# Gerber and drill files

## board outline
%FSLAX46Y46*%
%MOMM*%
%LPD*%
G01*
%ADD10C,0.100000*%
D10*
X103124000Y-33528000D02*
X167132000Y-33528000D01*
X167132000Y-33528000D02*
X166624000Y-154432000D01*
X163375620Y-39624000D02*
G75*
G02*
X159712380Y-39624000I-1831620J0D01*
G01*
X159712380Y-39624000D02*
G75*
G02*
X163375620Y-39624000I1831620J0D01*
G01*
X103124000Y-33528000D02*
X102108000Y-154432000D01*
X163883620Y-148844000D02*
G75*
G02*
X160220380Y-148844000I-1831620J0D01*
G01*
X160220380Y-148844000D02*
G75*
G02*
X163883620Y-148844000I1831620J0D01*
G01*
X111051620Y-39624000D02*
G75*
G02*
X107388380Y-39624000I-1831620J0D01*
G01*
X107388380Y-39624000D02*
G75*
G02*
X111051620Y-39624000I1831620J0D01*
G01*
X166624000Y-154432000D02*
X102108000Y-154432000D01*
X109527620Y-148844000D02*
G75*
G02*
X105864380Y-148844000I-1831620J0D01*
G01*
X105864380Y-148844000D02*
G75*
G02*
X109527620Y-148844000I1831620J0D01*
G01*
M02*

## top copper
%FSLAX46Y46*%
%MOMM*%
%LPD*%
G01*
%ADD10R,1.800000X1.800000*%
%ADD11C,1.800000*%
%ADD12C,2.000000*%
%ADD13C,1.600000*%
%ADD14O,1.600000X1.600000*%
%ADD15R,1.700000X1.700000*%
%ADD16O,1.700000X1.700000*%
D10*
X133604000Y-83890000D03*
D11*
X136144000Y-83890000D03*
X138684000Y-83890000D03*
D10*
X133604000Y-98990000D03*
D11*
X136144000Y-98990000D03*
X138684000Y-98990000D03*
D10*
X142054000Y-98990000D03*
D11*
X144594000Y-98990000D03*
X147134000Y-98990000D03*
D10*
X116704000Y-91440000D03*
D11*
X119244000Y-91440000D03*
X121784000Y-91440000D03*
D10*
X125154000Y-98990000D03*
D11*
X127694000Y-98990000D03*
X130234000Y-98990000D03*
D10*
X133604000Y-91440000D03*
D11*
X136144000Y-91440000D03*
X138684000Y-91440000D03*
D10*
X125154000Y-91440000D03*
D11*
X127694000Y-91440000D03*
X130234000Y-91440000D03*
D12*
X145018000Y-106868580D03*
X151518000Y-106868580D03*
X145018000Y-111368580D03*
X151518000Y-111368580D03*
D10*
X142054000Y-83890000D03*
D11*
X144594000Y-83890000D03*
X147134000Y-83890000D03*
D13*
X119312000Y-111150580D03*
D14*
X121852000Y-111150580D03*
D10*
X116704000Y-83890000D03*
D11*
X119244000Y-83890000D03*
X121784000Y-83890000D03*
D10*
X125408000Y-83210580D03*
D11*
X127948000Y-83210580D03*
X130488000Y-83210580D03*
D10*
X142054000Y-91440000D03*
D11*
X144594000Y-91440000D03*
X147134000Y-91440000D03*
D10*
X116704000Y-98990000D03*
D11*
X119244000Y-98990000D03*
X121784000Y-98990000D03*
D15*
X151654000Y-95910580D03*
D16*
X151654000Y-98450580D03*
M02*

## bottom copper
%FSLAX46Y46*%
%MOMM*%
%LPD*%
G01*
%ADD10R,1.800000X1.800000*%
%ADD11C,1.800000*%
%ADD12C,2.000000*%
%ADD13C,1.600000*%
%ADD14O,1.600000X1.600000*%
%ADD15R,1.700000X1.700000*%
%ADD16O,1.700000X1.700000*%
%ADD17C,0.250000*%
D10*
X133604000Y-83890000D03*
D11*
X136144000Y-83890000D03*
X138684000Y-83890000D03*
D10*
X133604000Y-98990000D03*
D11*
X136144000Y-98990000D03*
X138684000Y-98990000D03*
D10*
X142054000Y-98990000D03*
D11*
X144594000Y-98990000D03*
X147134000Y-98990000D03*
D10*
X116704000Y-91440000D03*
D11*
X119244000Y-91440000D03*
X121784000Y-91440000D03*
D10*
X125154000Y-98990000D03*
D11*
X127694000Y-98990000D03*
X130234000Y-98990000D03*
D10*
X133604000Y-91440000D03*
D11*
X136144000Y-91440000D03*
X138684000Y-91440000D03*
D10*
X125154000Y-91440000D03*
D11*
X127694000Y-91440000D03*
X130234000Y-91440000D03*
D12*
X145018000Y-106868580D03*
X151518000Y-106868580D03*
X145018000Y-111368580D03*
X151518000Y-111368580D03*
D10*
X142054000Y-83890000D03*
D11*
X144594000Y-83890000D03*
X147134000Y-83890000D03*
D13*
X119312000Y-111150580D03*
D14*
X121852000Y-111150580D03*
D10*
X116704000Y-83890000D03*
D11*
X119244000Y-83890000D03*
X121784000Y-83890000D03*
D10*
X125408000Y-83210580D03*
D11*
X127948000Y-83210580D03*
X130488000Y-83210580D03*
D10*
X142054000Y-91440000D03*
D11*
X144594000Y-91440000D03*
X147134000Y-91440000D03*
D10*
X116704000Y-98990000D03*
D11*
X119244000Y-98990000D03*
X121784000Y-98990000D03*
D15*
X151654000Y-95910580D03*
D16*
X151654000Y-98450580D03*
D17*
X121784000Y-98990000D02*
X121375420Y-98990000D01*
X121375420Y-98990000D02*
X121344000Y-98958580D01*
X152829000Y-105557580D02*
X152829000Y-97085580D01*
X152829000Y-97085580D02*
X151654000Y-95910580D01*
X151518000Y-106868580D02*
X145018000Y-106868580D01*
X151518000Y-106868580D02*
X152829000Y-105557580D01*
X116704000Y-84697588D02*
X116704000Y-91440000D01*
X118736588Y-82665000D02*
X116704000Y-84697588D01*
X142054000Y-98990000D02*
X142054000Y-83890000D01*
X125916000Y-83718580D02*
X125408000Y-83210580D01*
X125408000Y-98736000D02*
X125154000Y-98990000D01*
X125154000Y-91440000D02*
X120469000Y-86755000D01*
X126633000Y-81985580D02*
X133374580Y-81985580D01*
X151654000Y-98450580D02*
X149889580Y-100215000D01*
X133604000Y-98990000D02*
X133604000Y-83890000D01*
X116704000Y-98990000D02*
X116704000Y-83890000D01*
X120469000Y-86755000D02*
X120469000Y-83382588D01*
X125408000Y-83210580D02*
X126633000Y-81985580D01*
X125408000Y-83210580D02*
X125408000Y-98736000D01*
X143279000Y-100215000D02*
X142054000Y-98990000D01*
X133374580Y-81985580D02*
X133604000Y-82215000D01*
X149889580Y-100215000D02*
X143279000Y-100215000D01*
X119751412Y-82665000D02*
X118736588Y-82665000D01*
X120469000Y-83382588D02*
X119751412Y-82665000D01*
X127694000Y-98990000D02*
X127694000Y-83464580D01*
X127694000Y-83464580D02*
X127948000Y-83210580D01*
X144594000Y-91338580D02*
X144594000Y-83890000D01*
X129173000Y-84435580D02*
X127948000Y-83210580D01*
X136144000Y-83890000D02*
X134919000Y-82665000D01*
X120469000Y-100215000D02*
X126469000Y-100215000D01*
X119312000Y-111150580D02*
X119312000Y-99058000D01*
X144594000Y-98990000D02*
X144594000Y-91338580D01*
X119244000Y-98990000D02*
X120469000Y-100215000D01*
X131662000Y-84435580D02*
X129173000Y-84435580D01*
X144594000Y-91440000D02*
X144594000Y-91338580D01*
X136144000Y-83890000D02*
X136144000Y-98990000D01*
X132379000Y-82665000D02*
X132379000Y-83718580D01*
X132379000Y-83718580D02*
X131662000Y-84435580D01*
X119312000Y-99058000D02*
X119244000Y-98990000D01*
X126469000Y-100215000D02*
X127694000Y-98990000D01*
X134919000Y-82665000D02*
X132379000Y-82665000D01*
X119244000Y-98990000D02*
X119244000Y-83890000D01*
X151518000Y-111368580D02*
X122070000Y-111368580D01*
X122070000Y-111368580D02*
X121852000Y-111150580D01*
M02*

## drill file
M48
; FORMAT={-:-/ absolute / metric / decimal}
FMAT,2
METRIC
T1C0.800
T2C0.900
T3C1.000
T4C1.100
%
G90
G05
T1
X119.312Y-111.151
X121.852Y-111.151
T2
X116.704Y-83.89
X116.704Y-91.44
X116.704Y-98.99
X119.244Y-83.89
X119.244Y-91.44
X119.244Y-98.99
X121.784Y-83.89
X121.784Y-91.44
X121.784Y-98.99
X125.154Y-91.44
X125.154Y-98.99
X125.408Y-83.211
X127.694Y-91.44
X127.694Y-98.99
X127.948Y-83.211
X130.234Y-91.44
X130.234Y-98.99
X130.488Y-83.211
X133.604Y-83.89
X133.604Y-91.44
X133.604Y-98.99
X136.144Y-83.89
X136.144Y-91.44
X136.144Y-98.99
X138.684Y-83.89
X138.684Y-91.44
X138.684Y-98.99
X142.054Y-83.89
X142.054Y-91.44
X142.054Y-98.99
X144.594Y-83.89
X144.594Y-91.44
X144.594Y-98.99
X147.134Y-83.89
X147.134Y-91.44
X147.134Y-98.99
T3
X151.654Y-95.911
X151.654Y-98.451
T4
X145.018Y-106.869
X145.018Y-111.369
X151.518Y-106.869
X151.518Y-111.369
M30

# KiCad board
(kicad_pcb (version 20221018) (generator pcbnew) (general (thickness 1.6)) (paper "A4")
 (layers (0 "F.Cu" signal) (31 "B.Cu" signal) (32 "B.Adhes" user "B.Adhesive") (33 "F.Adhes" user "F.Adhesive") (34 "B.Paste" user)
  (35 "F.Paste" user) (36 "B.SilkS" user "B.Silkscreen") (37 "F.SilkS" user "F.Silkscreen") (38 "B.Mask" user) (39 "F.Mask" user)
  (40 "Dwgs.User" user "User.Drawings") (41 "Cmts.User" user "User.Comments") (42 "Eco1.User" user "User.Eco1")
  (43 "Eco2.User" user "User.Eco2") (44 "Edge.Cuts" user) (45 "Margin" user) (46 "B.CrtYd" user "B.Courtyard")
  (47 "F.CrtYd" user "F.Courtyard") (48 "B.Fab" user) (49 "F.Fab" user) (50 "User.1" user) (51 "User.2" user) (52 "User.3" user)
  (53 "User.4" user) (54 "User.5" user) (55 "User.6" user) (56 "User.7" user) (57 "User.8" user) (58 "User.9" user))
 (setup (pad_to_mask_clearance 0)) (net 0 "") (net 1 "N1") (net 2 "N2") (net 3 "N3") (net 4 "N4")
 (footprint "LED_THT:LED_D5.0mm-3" (layer "F.Cu") (at 133.604 83.89)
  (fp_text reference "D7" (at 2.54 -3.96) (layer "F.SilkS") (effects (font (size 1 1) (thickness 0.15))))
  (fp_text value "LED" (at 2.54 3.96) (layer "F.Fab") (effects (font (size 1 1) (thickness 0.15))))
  (pad "1" thru_hole rect (at 0 0) (size 1.8 1.8) (drill 0.9) (layers "*.Cu" "*.Mask") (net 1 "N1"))
  (pad "2" thru_hole circle (at 2.54 0) (size 1.8 1.8) (drill 0.9) (layers "*.Cu" "*.Mask") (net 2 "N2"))
  (pad "3" thru_hole circle (at 5.08 0) (size 1.8 1.8) (drill 0.9) (layers "*.Cu" "*.Mask")))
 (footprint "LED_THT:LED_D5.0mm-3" (layer "F.Cu") (at 133.604 98.99)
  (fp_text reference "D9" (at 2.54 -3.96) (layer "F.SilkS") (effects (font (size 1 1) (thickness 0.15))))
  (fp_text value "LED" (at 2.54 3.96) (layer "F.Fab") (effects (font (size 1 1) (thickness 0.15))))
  (pad "1" thru_hole rect (at 0 0) (size 1.8 1.8) (drill 0.9) (layers "*.Cu" "*.Mask") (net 1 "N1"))
  (pad "2" thru_hole circle (at 2.54 0) (size 1.8 1.8) (drill 0.9) (layers "*.Cu" "*.Mask") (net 2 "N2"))
  (pad "3" thru_hole circle (at 5.08 0) (size 1.8 1.8) (drill 0.9) (layers "*.Cu" "*.Mask")))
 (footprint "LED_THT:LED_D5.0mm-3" (layer "F.Cu") (at 142.054 98.99)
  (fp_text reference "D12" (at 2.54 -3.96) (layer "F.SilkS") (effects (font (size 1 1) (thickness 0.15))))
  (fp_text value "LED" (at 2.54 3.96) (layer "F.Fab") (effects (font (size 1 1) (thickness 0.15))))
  (pad "1" thru_hole rect (at 0 0) (size 1.8 1.8) (drill 0.9) (layers "*.Cu" "*.Mask") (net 1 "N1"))
  (pad "2" thru_hole circle (at 2.54 0) (size 1.8 1.8) (drill 0.9) (layers "*.Cu" "*.Mask") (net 2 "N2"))
  (pad "3" thru_hole circle (at 5.08 0) (size 1.8 1.8) (drill 0.9) (layers "*.Cu" "*.Mask")))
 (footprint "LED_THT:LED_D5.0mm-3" (layer "F.Cu") (at 116.704 91.44)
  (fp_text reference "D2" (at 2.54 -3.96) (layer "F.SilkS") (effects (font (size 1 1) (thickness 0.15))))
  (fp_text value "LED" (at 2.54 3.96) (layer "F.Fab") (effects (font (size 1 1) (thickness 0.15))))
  (pad "1" thru_hole rect (at 0 0) (size 1.8 1.8) (drill 0.9) (layers "*.Cu" "*.Mask") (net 1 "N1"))
  (pad "2" thru_hole circle (at 2.54 0) (size 1.8 1.8) (drill 0.9) (layers "*.Cu" "*.Mask") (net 2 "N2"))
  (pad "3" thru_hole circle (at 5.08 0) (size 1.8 1.8) (drill 0.9) (layers "*.Cu" "*.Mask")))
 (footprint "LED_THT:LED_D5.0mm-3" (layer "F.Cu") (at 125.154 98.99)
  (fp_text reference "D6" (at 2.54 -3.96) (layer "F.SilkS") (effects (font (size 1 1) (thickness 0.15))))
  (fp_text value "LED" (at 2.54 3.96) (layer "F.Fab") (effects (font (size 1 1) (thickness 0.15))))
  (pad "1" thru_hole rect (at 0 0) (size 1.8 1.8) (drill 0.9) (layers "*.Cu" "*.Mask") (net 1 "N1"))
  (pad "2" thru_hole circle (at 2.54 0) (size 1.8 1.8) (drill 0.9) (layers "*.Cu" "*.Mask") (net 2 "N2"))
  (pad "3" thru_hole circle (at 5.08 0) (size 1.8 1.8) (drill 0.9) (layers "*.Cu" "*.Mask")))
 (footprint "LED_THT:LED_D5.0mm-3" (layer "F.Cu") (at 133.604 91.44)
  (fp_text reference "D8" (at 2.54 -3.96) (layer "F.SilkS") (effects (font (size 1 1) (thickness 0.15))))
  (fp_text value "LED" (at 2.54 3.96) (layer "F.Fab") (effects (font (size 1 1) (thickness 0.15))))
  (pad "1" thru_hole rect (at 0 0) (size 1.8 1.8) (drill 0.9) (layers "*.Cu" "*.Mask") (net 1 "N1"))
  (pad "2" thru_hole circle (at 2.54 0) (size 1.8 1.8) (drill 0.9) (layers "*.Cu" "*.Mask") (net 2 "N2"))
  (pad "3" thru_hole circle (at 5.08 0) (size 1.8 1.8) (drill 0.9) (layers "*.Cu" "*.Mask")))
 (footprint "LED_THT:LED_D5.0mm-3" (layer "F.Cu") (at 125.154 91.44)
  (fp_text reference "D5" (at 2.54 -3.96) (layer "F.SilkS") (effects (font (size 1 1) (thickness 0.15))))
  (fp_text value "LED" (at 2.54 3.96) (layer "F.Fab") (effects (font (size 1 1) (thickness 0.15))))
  (pad "1" thru_hole rect (at 0 0) (size 1.8 1.8) (drill 0.9) (layers "*.Cu" "*.Mask") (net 1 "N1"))
  (pad "2" thru_hole circle (at 2.54 0) (size 1.8 1.8) (drill 0.9) (layers "*.Cu" "*.Mask") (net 2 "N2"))
  (pad "3" thru_hole circle (at 5.08 0) (size 1.8 1.8) (drill 0.9) (layers "*.Cu" "*.Mask")))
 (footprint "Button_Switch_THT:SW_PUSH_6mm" (layer "F.Cu") (at 145.018 106.86858)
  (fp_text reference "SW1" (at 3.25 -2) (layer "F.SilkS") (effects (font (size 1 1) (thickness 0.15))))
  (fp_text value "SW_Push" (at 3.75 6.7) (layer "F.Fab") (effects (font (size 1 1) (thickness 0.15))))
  (pad "1" thru_hole circle (at 0 0 90) (size 2 2) (drill 1.1) (layers "*.Cu" "*.Mask") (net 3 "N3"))
  (pad "1" thru_hole circle (at 6.5 0 90) (size 2 2) (drill 1.1) (layers "*.Cu" "*.Mask") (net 3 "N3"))
  (pad "2" thru_hole circle (at 0 4.5 90) (size 2 2) (drill 1.1) (layers "*.Cu" "*.Mask") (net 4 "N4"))
  (pad "2" thru_hole circle (at 6.5 4.5 90) (size 2 2) (drill 1.1) (layers "*.Cu" "*.Mask") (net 4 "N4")))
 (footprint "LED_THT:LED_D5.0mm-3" (layer "F.Cu") (at 142.054 83.89)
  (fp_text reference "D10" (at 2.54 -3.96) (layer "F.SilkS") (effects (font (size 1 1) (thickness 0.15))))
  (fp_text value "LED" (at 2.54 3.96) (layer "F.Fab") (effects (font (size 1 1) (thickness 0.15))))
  (pad "1" thru_hole rect (at 0 0) (size 1.8 1.8) (drill 0.9) (layers "*.Cu" "*.Mask") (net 1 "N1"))
  (pad "2" thru_hole circle (at 2.54 0) (size 1.8 1.8) (drill 0.9) (layers "*.Cu" "*.Mask") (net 2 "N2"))
  (pad "3" thru_hole circle (at 5.08 0) (size 1.8 1.8) (drill 0.9) (layers "*.Cu" "*.Mask")))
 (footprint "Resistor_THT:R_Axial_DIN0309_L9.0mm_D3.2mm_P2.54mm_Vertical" (layer "F.Cu") (at 119.312 111.15058)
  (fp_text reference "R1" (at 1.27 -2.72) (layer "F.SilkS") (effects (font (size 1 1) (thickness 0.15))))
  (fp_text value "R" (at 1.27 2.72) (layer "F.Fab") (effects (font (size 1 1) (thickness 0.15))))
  (pad "1" thru_hole circle (at 0 0) (size 1.6 1.6) (drill 0.8) (layers "*.Cu" "*.Mask") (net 2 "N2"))
  (pad "2" thru_hole oval (at 2.54 0) (size 1.6 1.6) (drill 0.8) (layers "*.Cu" "*.Mask") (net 4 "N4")))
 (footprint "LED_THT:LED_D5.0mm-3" (layer "F.Cu") (at 116.704 83.89)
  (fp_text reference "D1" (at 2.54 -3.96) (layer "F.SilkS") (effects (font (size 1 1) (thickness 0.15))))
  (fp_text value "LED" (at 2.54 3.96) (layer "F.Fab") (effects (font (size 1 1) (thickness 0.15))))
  (pad "1" thru_hole rect (at 0 0) (size 1.8 1.8) (drill 0.9) (layers "*.Cu" "*.Mask") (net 1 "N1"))
  (pad "2" thru_hole circle (at 2.54 0) (size 1.8 1.8) (drill 0.9) (layers "*.Cu" "*.Mask") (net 2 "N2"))
  (pad "3" thru_hole circle (at 5.08 0) (size 1.8 1.8) (drill 0.9) (layers "*.Cu" "*.Mask")))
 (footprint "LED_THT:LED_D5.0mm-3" (layer "F.Cu") (at 125.408 83.21058)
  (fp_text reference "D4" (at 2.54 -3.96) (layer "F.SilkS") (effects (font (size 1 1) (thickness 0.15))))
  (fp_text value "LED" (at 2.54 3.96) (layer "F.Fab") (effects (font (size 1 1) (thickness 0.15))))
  (pad "1" thru_hole rect (at 0 0) (size 1.8 1.8) (drill 0.9) (layers "*.Cu" "*.Mask") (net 1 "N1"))
  (pad "2" thru_hole circle (at 2.54 0) (size 1.8 1.8) (drill 0.9) (layers "*.Cu" "*.Mask") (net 2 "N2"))
  (pad "3" thru_hole circle (at 5.08 0) (size 1.8 1.8) (drill 0.9) (layers "*.Cu" "*.Mask")))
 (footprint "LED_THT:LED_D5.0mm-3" (layer "F.Cu") (at 142.054 91.44)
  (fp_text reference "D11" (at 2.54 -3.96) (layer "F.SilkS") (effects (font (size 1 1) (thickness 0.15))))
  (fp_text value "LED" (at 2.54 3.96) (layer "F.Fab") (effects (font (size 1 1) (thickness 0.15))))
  (pad "1" thru_hole rect (at 0 0) (size 1.8 1.8) (drill 0.9) (layers "*.Cu" "*.Mask") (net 1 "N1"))
  (pad "2" thru_hole circle (at 2.54 0) (size 1.8 1.8) (drill 0.9) (layers "*.Cu" "*.Mask") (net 2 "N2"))
  (pad "3" thru_hole circle (at 5.08 0) (size 1.8 1.8) (drill 0.9) (layers "*.Cu" "*.Mask")))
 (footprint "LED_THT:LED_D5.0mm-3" (layer "F.Cu") (at 116.704 98.99)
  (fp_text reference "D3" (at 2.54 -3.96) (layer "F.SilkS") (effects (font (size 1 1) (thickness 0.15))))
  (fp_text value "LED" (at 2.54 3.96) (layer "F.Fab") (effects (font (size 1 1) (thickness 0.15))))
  (pad "1" thru_hole rect (at 0 0) (size 1.8 1.8) (drill 0.9) (layers "*.Cu" "*.Mask") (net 1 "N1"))
  (pad "2" thru_hole circle (at 2.54 0) (size 1.8 1.8) (drill 0.9) (layers "*.Cu" "*.Mask") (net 2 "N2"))
  (pad "3" thru_hole circle (at 5.08 0) (size 1.8 1.8) (drill 0.9) (layers "*.Cu" "*.Mask")))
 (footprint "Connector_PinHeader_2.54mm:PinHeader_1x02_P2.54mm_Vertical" (layer "F.Cu") (at 151.654 95.91058)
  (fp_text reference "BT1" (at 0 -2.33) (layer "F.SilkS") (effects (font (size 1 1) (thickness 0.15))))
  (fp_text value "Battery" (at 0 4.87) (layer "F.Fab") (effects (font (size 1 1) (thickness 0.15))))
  (pad "1" thru_hole rect (at 0 0) (size 1.7 1.7) (drill 1) (layers "*.Cu" "*.Mask") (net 3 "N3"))
  (pad "2" thru_hole oval (at 0 2.54) (size 1.7 1.7) (drill 1) (layers "*.Cu" "*.Mask") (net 1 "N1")))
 (gr_line (start 103.124 33.528) (end 167.132 33.528) (stroke (width 0.1) (type default)) (layer "Edge.Cuts"))
 (gr_line (start 167.132 33.528) (end 166.624 154.432) (stroke (width 0.1) (type default)) (layer "Edge.Cuts"))
 (gr_circle (center 161.544 39.624) (end 160.02 38.608) (stroke (width 0.1) (type default)) (fill none) (layer "Edge.Cuts"))
 (gr_line (start 103.124 33.528) (end 102.108 154.432) (stroke (width 0.1) (type default)) (layer "Edge.Cuts"))
 (gr_circle (center 162.052 148.844) (end 161.036 147.32) (stroke (width 0.1) (type default)) (fill none) (layer "Edge.Cuts"))
 (gr_circle (center 109.22 39.624) (end 110.744 40.64) (stroke (width 0.1) (type default)) (fill none) (layer "Edge.Cuts"))
 (gr_line (start 166.624 154.432) (end 102.108 154.432) (stroke (width 0.1) (type default)) (layer "Edge.Cuts"))
 (gr_circle (center 107.696 148.844) (end 106.68 150.368) (stroke (width 0.1) (type default)) (fill none) (layer "Edge.Cuts"))
 (segment (start 121.784 98.99) (end 121.37542 98.99) (width 0.25) (layer "B.Cu") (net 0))
 (segment (start 121.37542 98.99) (end 121.344 98.95858) (width 0.25) (layer "B.Cu") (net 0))
 (segment (start 152.829 105.55758) (end 152.829 97.08558) (width 0.25) (layer "B.Cu") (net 3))
 (segment (start 152.829 97.08558) (end 151.654 95.91058) (width 0.25) (layer "B.Cu") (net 3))
 (segment (start 151.518 106.86858) (end 145.018 106.86858) (width 0.25) (layer "B.Cu") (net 3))
 (segment (start 151.518 106.86858) (end 152.829 105.55758) (width 0.25) (layer "B.Cu") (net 3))
 (segment (start 116.704 84.697588) (end 116.704 91.44) (width 0.25) (layer "B.Cu") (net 1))
 (segment (start 118.736588 82.665) (end 116.704 84.697588) (width 0.25) (layer "B.Cu") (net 1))
 (segment (start 142.054 98.99) (end 142.054 83.89) (width 0.25) (layer "B.Cu") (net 1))
 (segment (start 125.916 83.71858) (end 125.408 83.21058) (width 0.25) (layer "B.Cu") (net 1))
 (segment (start 125.408 98.736) (end 125.154 98.99) (width 0.25) (layer "B.Cu") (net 1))
 (segment (start 125.154 91.44) (end 120.469 86.755) (width 0.25) (layer "B.Cu") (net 1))
 (segment (start 126.633 81.98558) (end 133.37458 81.98558) (width 0.25) (layer "B.Cu") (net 1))
 (segment (start 151.654 98.45058) (end 149.88958 100.215) (width 0.25) (layer "B.Cu") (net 1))
 (segment (start 133.604 98.99) (end 133.604 83.89) (width 0.25) (layer "B.Cu") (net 1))
 (segment (start 116.704 98.99) (end 116.704 83.89) (width 0.25) (layer "B.Cu") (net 1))
 (segment (start 120.469 86.755) (end 120.469 83.382588) (width 0.25) (layer "B.Cu") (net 1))
 (segment (start 125.408 83.21058) (end 126.633 81.98558) (width 0.25) (layer "B.Cu") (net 1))
 (segment (start 125.408 83.21058) (end 125.408 98.736) (width 0.25) (layer "B.Cu") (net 1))
 (segment (start 143.279 100.215) (end 142.054 98.99) (width 0.25) (layer "B.Cu") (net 1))
 (segment (start 133.37458 81.98558) (end 133.604 82.215) (width 0.25) (layer "B.Cu") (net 1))
 (segment (start 149.88958 100.215) (end 143.279 100.215) (width 0.25) (layer "B.Cu") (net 1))
 (segment (start 119.751412 82.665) (end 118.736588 82.665) (width 0.25) (layer "B.Cu") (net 1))
 (segment (start 120.469 83.382588) (end 119.751412 82.665) (width 0.25) (layer "B.Cu") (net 1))
 (segment (start 127.694 98.99) (end 127.694 83.46458) (width 0.25) (layer "B.Cu") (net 2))
 (segment (start 127.694 83.46458) (end 127.948 83.21058) (width 0.25) (layer "B.Cu") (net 2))
 (segment (start 144.594 91.33858) (end 144.594 83.89) (width 0.25) (layer "B.Cu") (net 2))
 (segment (start 129.173 84.43558) (end 127.948 83.21058) (width 0.25) (layer "B.Cu") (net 2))
 (segment (start 136.144 83.89) (end 134.919 82.665) (width 0.25) (layer "B.Cu") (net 2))
 (segment (start 120.469 100.215) (end 126.469 100.215) (width 0.25) (layer "B.Cu") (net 2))
 (segment (start 119.312 111.15058) (end 119.312 99.058) (width 0.25) (layer "B.Cu") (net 2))
 (segment (start 144.594 98.99) (end 144.594 91.33858) (width 0.25) (layer "B.Cu") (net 2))
 (segment (start 119.244 98.99) (end 120.469 100.215) (width 0.25) (layer "B.Cu") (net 2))
 (segment (start 131.662 84.43558) (end 129.173 84.43558) (width 0.25) (layer "B.Cu") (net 2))
 (segment (start 144.594 91.44) (end 144.594 91.33858) (width 0.25) (layer "B.Cu") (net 2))
 (segment (start 136.144 83.89) (end 136.144 98.99) (width 0.25) (layer "B.Cu") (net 2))
 (segment (start 132.379 82.665) (end 132.379 83.71858) (width 0.25) (layer "B.Cu") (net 2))
 (segment (start 132.379 83.71858) (end 131.662 84.43558) (width 0.25) (layer "B.Cu") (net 2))
 (segment (start 119.312 99.058) (end 119.244 98.99) (width 0.25) (layer "B.Cu") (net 2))
 (segment (start 126.469 100.215) (end 127.694 98.99) (width 0.25) (layer "B.Cu") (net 2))
 (segment (start 134.919 82.665) (end 132.379 82.665) (width 0.25) (layer "B.Cu") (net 2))
 (segment (start 119.244 98.99) (end 119.244 83.89) (width 0.25) (layer "B.Cu") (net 2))
 (segment (start 151.518 111.36858) (end 122.07 111.36858) (width 0.25) (layer "B.Cu") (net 4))
 (segment (start 122.07 111.36858) (end 121.852 111.15058) (width 0.25) (layer "B.Cu") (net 4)))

